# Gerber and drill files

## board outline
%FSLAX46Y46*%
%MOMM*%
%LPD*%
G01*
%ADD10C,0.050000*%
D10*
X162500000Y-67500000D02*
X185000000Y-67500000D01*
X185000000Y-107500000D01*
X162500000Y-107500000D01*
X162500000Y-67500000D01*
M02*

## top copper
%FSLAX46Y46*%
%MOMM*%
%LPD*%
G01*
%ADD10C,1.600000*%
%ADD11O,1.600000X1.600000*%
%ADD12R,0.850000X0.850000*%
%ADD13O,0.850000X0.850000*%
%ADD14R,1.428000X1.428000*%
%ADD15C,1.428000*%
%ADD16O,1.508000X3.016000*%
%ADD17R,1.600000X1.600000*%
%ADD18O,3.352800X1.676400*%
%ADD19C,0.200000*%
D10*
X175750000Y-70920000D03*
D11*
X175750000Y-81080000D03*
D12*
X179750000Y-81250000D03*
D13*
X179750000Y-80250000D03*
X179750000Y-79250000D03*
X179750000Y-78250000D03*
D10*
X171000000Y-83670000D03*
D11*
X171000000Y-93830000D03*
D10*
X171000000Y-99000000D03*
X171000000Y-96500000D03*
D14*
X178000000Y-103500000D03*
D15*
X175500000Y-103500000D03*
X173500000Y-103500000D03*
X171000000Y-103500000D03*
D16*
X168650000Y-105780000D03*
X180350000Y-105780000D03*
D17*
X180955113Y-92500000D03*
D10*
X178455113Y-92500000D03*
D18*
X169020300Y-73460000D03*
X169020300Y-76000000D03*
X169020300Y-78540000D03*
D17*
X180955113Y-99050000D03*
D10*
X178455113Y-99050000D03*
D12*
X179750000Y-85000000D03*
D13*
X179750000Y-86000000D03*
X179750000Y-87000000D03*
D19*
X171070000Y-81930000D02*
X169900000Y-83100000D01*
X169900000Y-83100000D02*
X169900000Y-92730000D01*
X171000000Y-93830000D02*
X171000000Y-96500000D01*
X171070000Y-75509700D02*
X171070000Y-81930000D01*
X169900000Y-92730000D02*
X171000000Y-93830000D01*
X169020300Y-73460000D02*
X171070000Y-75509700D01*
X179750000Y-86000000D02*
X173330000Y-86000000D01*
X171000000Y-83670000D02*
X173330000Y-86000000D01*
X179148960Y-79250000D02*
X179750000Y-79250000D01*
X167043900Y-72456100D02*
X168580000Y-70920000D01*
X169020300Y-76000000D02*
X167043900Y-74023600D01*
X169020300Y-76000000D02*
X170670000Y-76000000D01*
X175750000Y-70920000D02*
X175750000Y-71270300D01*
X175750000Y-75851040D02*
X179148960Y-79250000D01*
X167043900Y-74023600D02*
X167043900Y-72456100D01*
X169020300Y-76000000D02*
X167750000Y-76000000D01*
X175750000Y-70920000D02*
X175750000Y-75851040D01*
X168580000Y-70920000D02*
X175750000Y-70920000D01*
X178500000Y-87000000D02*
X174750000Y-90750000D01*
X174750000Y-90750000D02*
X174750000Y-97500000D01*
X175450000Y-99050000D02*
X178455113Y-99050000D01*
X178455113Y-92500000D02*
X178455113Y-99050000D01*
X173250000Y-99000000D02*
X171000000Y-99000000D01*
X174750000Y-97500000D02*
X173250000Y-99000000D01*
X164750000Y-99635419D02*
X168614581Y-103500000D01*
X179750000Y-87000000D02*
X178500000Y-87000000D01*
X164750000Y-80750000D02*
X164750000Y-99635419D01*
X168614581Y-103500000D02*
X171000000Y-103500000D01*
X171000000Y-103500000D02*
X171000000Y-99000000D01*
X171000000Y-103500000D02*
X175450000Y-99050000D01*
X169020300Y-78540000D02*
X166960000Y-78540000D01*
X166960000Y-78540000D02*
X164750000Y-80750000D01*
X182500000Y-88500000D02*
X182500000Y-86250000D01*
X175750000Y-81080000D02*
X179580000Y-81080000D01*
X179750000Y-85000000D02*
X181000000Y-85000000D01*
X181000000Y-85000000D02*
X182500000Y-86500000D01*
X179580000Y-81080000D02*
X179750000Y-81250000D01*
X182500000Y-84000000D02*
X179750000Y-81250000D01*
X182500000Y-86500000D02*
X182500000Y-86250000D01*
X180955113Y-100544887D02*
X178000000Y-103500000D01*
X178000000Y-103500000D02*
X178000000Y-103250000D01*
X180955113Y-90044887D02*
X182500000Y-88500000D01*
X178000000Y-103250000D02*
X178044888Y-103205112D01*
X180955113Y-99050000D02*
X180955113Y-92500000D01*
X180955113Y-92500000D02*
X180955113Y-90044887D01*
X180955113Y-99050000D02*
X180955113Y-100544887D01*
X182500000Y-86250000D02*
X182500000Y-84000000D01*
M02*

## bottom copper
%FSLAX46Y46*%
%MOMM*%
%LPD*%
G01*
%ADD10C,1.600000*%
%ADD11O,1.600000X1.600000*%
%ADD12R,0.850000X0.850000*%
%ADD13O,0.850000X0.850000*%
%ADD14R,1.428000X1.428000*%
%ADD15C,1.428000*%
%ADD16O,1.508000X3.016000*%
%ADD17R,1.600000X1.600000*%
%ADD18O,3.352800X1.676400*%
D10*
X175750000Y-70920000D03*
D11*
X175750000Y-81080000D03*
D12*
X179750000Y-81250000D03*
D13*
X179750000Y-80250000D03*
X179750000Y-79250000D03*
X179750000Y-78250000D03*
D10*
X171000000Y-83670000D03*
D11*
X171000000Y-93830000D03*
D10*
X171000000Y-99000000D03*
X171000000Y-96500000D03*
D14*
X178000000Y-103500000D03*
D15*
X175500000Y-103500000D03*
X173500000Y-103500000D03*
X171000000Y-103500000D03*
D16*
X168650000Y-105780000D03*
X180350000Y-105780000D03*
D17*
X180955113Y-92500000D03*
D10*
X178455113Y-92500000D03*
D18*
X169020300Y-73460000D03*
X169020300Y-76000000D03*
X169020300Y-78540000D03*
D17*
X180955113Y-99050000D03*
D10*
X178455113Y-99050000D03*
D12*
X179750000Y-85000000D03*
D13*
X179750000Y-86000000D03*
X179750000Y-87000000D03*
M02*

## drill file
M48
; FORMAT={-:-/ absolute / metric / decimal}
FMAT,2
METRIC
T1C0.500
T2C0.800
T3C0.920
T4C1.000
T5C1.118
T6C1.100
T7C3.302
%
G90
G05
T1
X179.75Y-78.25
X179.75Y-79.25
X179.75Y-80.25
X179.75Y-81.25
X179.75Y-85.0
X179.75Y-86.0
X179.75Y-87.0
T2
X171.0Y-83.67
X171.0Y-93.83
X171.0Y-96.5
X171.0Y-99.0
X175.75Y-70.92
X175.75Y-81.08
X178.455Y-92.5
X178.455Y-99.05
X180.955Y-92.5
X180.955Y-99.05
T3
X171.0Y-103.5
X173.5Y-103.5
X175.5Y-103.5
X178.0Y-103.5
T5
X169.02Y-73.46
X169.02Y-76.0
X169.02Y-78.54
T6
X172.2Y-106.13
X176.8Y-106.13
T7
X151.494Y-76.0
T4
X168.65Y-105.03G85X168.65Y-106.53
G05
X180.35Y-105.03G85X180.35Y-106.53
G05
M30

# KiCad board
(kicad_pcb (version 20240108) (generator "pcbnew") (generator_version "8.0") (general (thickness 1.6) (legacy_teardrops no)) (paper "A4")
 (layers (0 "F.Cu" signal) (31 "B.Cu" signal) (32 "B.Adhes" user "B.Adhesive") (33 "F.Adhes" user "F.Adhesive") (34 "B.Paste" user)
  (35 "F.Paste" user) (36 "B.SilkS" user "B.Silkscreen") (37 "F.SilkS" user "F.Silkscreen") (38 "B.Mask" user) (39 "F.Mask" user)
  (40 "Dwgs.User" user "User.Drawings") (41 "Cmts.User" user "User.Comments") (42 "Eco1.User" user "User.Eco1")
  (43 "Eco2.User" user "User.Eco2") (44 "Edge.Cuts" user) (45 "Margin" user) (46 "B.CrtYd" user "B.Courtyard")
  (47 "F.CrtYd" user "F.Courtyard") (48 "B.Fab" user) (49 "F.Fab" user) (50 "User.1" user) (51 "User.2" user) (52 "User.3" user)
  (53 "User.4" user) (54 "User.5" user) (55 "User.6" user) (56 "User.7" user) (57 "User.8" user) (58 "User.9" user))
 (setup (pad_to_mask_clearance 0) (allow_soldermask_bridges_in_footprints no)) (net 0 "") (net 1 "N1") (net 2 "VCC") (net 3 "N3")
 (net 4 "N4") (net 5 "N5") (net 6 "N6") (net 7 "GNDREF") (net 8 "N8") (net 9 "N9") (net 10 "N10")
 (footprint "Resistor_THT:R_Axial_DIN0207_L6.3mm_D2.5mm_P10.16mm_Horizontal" (layer "F.Cu") (at 175.75 70.92 -90)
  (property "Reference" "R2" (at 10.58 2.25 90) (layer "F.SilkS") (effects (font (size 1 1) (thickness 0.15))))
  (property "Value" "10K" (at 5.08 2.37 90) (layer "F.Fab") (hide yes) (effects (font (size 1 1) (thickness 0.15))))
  (pad "1" thru_hole circle (at 0 0 270) (size 1.6 1.6) (drill 0.8) (layers "*.Cu" "*.Mask") (remove_unused_layers no) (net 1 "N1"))
  (pad "2" thru_hole oval (at 10.16 0 270) (size 1.6 1.6) (drill 0.8) (layers "*.Cu" "*.Mask") (remove_unused_layers no) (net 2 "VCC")))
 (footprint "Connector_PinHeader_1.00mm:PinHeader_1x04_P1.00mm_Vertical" (layer "F.Cu") (at 179.75 81.25 180)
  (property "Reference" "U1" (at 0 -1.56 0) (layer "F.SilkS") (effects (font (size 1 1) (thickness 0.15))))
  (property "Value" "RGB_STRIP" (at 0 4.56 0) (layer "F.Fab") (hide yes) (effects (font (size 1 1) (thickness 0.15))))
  (pad "1" thru_hole rect (at 0 0 180) (size 0.85 0.85) (drill 0.5) (layers "*.Cu" "*.Mask") (remove_unused_layers no) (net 2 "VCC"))
  (pad "2" thru_hole oval (at 0 1 180) (size 0.85 0.85) (drill 0.5) (layers "*.Cu" "*.Mask") (remove_unused_layers no) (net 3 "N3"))
  (pad "3" thru_hole oval (at 0 2 180) (size 0.85 0.85) (drill 0.5) (layers "*.Cu" "*.Mask") (remove_unused_layers no) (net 1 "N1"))
  (pad "4" thru_hole oval (at 0 3 180) (size 0.85 0.85) (drill 0.5) (layers "*.Cu" "*.Mask") (remove_unused_layers no) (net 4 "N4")))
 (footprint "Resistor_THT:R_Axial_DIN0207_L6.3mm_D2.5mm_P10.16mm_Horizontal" (layer "F.Cu") (at 171 83.67 -90)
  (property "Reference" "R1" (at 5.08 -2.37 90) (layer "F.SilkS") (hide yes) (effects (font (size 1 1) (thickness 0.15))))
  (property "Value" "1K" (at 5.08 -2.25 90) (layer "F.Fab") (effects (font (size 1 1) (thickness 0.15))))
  (pad "1" thru_hole circle (at 0 0 270) (size 1.6 1.6) (drill 0.8) (layers "*.Cu" "*.Mask") (remove_unused_layers no) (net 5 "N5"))
  (pad "2" thru_hole oval (at 10.16 0 270) (size 1.6 1.6) (drill 0.8) (layers "*.Cu" "*.Mask") (remove_unused_layers no) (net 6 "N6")))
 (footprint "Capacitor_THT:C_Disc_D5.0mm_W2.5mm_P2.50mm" (layer "F.Cu") (at 171 99 90)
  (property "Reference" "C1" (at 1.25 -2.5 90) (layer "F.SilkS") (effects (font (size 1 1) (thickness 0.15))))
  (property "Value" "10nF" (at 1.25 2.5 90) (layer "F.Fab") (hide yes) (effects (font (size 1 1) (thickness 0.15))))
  (pad "1" thru_hole circle (at 0 0 90) (size 1.6 1.6) (drill 0.8) (layers "*.Cu" "*.Mask") (remove_unused_layers no) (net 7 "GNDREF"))
  (pad "2" thru_hole circle (at 2.5 0 90) (size 1.6 1.6) (drill 0.8) (layers "*.Cu" "*.Mask") (remove_unused_layers no) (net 6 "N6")))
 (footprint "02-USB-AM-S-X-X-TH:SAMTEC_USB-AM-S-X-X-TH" (layer "F.Cu") (at 174.5 105.78)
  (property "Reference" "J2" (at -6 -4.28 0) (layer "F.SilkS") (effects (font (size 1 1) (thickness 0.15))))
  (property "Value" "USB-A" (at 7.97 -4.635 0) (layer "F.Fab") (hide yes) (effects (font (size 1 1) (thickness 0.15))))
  (pad "" np_thru_hole circle (at -2.3 0.35) (size 1.1 1.1) (drill 1.1) (layers "*.Cu" "*.Mask"))
  (pad "" np_thru_hole circle (at 2.3 0.35) (size 1.1 1.1) (drill 1.1) (layers "*.Cu" "*.Mask"))
  (pad "01" thru_hole rect (at 3.5 -2.28) (size 1.428 1.428) (drill 0.92) (layers "*.Cu" "*.Mask") (remove_unused_layers no) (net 2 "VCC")
   (solder_mask_margin 0.102))
  (pad "02" thru_hole circle (at 1 -2.28) (size 1.428 1.428) (drill 0.92) (layers "*.Cu" "*.Mask") (remove_unused_layers no) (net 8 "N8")
   (solder_mask_margin 0.102))
  (pad "03" thru_hole circle (at -1 -2.28) (size 1.428 1.428) (drill 0.92) (layers "*.Cu" "*.Mask") (remove_unused_layers no) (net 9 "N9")
   (solder_mask_margin 0.102))
  (pad "04" thru_hole circle (at -3.5 -2.28) (size 1.428 1.428) (drill 0.92) (layers "*.Cu" "*.Mask") (remove_unused_layers no)
   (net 7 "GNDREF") (solder_mask_margin 0.102))
  (pad "S1" thru_hole oval (at -5.85 0) (size 1.508 3.016) (drill oval 1 2.5) (layers "*.Cu" "*.Mask") (remove_unused_layers no)
   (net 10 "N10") (solder_mask_margin 0.102))
  (pad "S2" thru_hole oval (at 5.85 0) (size 1.508 3.016) (drill oval 1 2.5) (layers "*.Cu" "*.Mask") (remove_unused_layers no)
   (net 10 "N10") (solder_mask_margin 0.102)))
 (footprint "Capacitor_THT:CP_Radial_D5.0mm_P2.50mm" (layer "B.Cu") (at 180.955113 92.5 180)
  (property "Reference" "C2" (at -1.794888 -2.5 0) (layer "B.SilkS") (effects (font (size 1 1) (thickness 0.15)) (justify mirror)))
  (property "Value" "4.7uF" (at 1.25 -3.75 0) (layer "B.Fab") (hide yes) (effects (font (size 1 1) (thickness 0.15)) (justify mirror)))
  (pad "1" thru_hole rect (at 0 0 180) (size 1.6 1.6) (drill 0.8) (layers "*.Cu" "*.Mask") (remove_unused_layers no) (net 2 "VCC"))
  (pad "2" thru_hole circle (at 2.5 0 180) (size 1.6 1.6) (drill 0.8) (layers "*.Cu" "*.Mask") (remove_unused_layers no) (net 7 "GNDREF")))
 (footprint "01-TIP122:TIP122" (layer "B.Cu") (at 162.6703 76 -90)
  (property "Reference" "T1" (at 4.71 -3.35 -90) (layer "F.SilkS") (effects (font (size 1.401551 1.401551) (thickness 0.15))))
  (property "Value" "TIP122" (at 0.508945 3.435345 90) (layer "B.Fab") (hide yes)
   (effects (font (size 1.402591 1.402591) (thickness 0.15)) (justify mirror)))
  (pad "" np_thru_hole circle (at 0 11.176 270) (size 3.302 3.302) (drill 3.302) (layers "*.Cu" "*.Mask"))
  (pad "1" thru_hole oval (at -2.54 -6.35 270) (size 1.6764 3.3528) (drill 1.1176) (layers "*.Cu" "*.Mask") (remove_unused_layers no)
   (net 6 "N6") (solder_mask_margin 0.102))
  (pad "2" thru_hole oval (at 0 -6.35 270) (size 1.6764 3.3528) (drill 1.1176) (layers "*.Cu" "*.Mask") (remove_unused_layers no)
   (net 1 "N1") (solder_mask_margin 0.102))
  (pad "3" thru_hole oval (at 2.54 -6.35 270) (size 1.6764 3.3528) (drill 1.1176) (layers "*.Cu" "*.Mask") (remove_unused_layers no)
   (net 7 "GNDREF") (solder_mask_margin 0.102))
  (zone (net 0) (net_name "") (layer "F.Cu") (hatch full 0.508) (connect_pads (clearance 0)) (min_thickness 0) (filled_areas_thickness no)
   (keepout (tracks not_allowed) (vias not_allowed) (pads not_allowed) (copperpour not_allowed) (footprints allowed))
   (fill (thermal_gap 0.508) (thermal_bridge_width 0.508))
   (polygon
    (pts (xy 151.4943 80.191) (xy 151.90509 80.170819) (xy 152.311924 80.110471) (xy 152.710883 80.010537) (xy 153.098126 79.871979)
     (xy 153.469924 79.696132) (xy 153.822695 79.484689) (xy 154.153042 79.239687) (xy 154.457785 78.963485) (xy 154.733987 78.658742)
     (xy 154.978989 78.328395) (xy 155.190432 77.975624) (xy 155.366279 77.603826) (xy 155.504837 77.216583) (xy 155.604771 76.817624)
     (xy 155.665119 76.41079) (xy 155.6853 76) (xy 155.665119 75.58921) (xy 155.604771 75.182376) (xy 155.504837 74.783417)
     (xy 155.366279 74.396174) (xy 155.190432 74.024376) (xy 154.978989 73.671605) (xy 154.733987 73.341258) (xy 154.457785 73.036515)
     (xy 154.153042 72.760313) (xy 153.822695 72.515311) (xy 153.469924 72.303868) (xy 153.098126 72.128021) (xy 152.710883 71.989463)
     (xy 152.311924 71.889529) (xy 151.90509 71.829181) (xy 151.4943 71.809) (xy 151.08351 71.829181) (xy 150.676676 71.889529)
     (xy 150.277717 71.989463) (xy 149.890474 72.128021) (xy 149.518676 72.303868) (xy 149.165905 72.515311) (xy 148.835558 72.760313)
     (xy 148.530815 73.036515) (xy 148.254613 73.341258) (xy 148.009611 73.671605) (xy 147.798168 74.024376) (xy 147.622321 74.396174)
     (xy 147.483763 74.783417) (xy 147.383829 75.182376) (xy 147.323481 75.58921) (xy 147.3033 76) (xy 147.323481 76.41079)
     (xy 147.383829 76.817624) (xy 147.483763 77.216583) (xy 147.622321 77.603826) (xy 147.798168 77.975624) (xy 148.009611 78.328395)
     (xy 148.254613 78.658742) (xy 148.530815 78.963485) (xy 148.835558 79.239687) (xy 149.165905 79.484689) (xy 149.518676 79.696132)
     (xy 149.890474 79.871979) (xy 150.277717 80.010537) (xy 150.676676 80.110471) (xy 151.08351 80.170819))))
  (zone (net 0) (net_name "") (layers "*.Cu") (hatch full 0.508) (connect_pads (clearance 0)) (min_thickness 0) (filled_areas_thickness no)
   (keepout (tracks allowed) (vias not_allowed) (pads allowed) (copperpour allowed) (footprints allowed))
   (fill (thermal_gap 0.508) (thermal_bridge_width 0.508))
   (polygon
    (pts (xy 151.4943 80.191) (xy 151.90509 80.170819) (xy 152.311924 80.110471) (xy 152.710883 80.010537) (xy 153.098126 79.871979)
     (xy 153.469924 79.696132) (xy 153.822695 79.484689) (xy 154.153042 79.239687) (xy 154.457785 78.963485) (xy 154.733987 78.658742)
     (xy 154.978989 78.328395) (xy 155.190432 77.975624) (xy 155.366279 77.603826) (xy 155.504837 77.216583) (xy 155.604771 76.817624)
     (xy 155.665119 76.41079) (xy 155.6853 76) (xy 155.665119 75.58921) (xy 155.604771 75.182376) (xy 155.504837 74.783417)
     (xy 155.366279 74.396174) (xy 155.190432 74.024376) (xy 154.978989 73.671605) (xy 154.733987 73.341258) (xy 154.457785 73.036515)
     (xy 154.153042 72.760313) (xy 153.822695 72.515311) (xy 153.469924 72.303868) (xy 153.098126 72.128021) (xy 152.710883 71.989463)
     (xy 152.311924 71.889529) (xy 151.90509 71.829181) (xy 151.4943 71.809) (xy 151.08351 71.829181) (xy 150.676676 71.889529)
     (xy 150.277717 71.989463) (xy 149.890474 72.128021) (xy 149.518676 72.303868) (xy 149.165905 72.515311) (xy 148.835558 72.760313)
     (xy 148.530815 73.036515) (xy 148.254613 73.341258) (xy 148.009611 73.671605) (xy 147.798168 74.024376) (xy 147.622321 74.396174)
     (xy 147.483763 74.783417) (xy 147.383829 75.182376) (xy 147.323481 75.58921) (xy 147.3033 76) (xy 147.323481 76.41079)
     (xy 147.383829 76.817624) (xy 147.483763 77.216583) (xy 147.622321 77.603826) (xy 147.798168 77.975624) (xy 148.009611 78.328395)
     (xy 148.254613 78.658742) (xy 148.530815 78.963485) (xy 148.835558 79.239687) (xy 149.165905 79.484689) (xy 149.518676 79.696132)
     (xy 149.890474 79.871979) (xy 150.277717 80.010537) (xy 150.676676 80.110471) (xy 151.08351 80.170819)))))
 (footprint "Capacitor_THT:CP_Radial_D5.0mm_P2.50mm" (layer "B.Cu") (at 180.955113 99.05 180)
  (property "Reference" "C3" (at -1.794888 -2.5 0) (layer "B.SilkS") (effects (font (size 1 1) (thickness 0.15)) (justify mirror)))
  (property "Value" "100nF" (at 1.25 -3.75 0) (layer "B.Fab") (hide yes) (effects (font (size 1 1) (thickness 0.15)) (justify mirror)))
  (pad "1" thru_hole rect (at 0 0 180) (size 1.6 1.6) (drill 0.8) (layers "*.Cu" "*.Mask") (remove_unused_layers no) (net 2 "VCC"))
  (pad "2" thru_hole circle (at 2.5 0 180) (size 1.6 1.6) (drill 0.8) (layers "*.Cu" "*.Mask") (remove_unused_layers no) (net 7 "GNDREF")))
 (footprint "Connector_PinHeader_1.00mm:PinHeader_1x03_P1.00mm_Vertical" (layer "B.Cu") (at 179.75 85 180)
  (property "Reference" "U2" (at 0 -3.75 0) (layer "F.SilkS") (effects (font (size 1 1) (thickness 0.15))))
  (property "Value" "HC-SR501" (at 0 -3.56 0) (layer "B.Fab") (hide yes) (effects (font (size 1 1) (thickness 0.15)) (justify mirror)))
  (pad "1" thru_hole rect (at 0 0 180) (size 0.85 0.85) (drill 0.5) (layers "*.Cu" "*.Mask") (remove_unused_layers no) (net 2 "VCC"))
  (pad "2" thru_hole oval (at 0 -1 180) (size 0.85 0.85) (drill 0.5) (layers "*.Cu" "*.Mask") (remove_unused_layers no) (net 5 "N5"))
  (pad "3" thru_hole oval (at 0 -2 180) (size 0.85 0.85) (drill 0.5) (layers "*.Cu" "*.Mask") (remove_unused_layers no) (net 7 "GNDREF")))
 (gr_rect (start 162.5 67.5) (end 185 107.5) (stroke (width 0.05) (type default)) (fill none) (layer "Edge.Cuts"))
 (segment (start 171.07 81.93) (end 169.9 83.1) (width 0.2) (layer "F.Cu") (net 6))
 (segment (start 169.9 83.1) (end 169.9 92.73) (width 0.2) (layer "F.Cu") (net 6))
 (segment (start 171 93.83) (end 171 96.5) (width 0.2) (layer "F.Cu") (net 6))
 (segment (start 171.07 75.5097) (end 171.07 81.93) (width 0.2) (layer "F.Cu") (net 6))
 (segment (start 169.9 92.73) (end 171 93.83) (width 0.2) (layer "F.Cu") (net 6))
 (segment (start 169.0203 73.46) (end 171.07 75.5097) (width 0.2) (layer "F.Cu") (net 6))
 (segment (start 179.75 86) (end 173.33 86) (width 0.2) (layer "F.Cu") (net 5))
 (segment (start 171 83.67) (end 173.33 86) (width 0.2) (layer "F.Cu") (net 5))
 (segment (start 179.14896 79.25) (end 179.75 79.25) (width 0.2) (layer "F.Cu") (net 1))
 (segment (start 167.0439 72.4561) (end 168.58 70.92) (width 0.2) (layer "F.Cu") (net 1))
 (segment (start 169.0203 76) (end 167.0439 74.0236) (width 0.2) (layer "F.Cu") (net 1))
 (segment (start 169.0203 76) (end 170.67 76) (width 0.2) (layer "F.Cu") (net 1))
 (segment (start 175.75 70.92) (end 175.75 71.2703) (width 0.2) (layer "F.Cu") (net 1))
 (segment (start 175.75 75.85104) (end 179.14896 79.25) (width 0.2) (layer "F.Cu") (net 1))
 (segment (start 167.0439 74.0236) (end 167.0439 72.4561) (width 0.2) (layer "F.Cu") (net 1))
 (segment (start 169.0203 76) (end 167.75 76) (width 0.2) (layer "F.Cu") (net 1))
 (segment (start 175.75 70.92) (end 175.75 75.85104) (width 0.2) (layer "F.Cu") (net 1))
 (segment (start 168.58 70.92) (end 175.75 70.92) (width 0.2) (layer "F.Cu") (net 1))
 (segment (start 178.5 87) (end 174.75 90.75) (width 0.2) (layer "F.Cu") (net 7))
 (segment (start 174.75 90.75) (end 174.75 97.5) (width 0.2) (layer "F.Cu") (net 7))
 (segment (start 175.45 99.05) (end 178.455113 99.05) (width 0.2) (layer "F.Cu") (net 7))
 (segment (start 178.455113 92.5) (end 178.455113 99.05) (width 0.2) (layer "F.Cu") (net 7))
 (segment (start 173.25 99) (end 171 99) (width 0.2) (layer "F.Cu") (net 7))
 (segment (start 174.75 97.5) (end 173.25 99) (width 0.2) (layer "F.Cu") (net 7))
 (segment (start 164.75 99.635419) (end 168.614581 103.5) (width 0.2) (layer "F.Cu") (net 7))
 (segment (start 179.75 87) (end 178.5 87) (width 0.2) (layer "F.Cu") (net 7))
 (segment (start 164.75 80.75) (end 164.75 99.635419) (width 0.2) (layer "F.Cu") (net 7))
 (segment (start 168.614581 103.5) (end 171 103.5) (width 0.2) (layer "F.Cu") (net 7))
 (segment (start 171 103.5) (end 171 99) (width 0.2) (layer "F.Cu") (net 7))
 (segment (start 171 103.5) (end 175.45 99.05) (width 0.2) (layer "F.Cu") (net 7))
 (segment (start 169.0203 78.54) (end 166.96 78.54) (width 0.2) (layer "F.Cu") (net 7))
 (segment (start 166.96 78.54) (end 164.75 80.75) (width 0.2) (layer "F.Cu") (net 7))
 (segment (start 182.5 88.5) (end 182.5 86.25) (width 0.2) (layer "F.Cu") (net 2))
 (segment (start 175.75 81.08) (end 179.58 81.08) (width 0.2) (layer "F.Cu") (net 2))
 (segment (start 179.75 85) (end 181 85) (width 0.2) (layer "F.Cu") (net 2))
 (segment (start 181 85) (end 182.5 86.5) (width 0.2) (layer "F.Cu") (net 2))
 (segment (start 179.58 81.08) (end 179.75 81.25) (width 0.2) (layer "F.Cu") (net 2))
 (segment (start 182.5 84) (end 179.75 81.25) (width 0.2) (layer "F.Cu") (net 2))
 (segment (start 182.5 86.5) (end 182.5 86.25) (width 0.2) (layer "F.Cu") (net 2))
 (segment (start 180.955113 100.544887) (end 178 103.5) (width 0.2) (layer "F.Cu") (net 2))
 (segment (start 178 103.5) (end 178 103.25) (width 0.2) (layer "F.Cu") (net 2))
 (segment (start 180.955113 90.044887) (end 182.5 88.5) (width 0.2) (layer "F.Cu") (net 2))
 (segment (start 178 103.25) (end 178.044888 103.205112) (width 0.2) (layer "F.Cu") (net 2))
 (segment (start 180.955113 99.05) (end 180.955113 92.5) (width 0.2) (layer "F.Cu") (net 2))
 (segment (start 180.955113 92.5) (end 180.955113 90.044887) (width 0.2) (layer "F.Cu") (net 2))
 (segment (start 180.955113 99.05) (end 180.955113 100.544887) (width 0.2) (layer "F.Cu") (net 2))
 (segment (start 182.5 86.25) (end 182.5 84) (width 0.2) (layer "F.Cu") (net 2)))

